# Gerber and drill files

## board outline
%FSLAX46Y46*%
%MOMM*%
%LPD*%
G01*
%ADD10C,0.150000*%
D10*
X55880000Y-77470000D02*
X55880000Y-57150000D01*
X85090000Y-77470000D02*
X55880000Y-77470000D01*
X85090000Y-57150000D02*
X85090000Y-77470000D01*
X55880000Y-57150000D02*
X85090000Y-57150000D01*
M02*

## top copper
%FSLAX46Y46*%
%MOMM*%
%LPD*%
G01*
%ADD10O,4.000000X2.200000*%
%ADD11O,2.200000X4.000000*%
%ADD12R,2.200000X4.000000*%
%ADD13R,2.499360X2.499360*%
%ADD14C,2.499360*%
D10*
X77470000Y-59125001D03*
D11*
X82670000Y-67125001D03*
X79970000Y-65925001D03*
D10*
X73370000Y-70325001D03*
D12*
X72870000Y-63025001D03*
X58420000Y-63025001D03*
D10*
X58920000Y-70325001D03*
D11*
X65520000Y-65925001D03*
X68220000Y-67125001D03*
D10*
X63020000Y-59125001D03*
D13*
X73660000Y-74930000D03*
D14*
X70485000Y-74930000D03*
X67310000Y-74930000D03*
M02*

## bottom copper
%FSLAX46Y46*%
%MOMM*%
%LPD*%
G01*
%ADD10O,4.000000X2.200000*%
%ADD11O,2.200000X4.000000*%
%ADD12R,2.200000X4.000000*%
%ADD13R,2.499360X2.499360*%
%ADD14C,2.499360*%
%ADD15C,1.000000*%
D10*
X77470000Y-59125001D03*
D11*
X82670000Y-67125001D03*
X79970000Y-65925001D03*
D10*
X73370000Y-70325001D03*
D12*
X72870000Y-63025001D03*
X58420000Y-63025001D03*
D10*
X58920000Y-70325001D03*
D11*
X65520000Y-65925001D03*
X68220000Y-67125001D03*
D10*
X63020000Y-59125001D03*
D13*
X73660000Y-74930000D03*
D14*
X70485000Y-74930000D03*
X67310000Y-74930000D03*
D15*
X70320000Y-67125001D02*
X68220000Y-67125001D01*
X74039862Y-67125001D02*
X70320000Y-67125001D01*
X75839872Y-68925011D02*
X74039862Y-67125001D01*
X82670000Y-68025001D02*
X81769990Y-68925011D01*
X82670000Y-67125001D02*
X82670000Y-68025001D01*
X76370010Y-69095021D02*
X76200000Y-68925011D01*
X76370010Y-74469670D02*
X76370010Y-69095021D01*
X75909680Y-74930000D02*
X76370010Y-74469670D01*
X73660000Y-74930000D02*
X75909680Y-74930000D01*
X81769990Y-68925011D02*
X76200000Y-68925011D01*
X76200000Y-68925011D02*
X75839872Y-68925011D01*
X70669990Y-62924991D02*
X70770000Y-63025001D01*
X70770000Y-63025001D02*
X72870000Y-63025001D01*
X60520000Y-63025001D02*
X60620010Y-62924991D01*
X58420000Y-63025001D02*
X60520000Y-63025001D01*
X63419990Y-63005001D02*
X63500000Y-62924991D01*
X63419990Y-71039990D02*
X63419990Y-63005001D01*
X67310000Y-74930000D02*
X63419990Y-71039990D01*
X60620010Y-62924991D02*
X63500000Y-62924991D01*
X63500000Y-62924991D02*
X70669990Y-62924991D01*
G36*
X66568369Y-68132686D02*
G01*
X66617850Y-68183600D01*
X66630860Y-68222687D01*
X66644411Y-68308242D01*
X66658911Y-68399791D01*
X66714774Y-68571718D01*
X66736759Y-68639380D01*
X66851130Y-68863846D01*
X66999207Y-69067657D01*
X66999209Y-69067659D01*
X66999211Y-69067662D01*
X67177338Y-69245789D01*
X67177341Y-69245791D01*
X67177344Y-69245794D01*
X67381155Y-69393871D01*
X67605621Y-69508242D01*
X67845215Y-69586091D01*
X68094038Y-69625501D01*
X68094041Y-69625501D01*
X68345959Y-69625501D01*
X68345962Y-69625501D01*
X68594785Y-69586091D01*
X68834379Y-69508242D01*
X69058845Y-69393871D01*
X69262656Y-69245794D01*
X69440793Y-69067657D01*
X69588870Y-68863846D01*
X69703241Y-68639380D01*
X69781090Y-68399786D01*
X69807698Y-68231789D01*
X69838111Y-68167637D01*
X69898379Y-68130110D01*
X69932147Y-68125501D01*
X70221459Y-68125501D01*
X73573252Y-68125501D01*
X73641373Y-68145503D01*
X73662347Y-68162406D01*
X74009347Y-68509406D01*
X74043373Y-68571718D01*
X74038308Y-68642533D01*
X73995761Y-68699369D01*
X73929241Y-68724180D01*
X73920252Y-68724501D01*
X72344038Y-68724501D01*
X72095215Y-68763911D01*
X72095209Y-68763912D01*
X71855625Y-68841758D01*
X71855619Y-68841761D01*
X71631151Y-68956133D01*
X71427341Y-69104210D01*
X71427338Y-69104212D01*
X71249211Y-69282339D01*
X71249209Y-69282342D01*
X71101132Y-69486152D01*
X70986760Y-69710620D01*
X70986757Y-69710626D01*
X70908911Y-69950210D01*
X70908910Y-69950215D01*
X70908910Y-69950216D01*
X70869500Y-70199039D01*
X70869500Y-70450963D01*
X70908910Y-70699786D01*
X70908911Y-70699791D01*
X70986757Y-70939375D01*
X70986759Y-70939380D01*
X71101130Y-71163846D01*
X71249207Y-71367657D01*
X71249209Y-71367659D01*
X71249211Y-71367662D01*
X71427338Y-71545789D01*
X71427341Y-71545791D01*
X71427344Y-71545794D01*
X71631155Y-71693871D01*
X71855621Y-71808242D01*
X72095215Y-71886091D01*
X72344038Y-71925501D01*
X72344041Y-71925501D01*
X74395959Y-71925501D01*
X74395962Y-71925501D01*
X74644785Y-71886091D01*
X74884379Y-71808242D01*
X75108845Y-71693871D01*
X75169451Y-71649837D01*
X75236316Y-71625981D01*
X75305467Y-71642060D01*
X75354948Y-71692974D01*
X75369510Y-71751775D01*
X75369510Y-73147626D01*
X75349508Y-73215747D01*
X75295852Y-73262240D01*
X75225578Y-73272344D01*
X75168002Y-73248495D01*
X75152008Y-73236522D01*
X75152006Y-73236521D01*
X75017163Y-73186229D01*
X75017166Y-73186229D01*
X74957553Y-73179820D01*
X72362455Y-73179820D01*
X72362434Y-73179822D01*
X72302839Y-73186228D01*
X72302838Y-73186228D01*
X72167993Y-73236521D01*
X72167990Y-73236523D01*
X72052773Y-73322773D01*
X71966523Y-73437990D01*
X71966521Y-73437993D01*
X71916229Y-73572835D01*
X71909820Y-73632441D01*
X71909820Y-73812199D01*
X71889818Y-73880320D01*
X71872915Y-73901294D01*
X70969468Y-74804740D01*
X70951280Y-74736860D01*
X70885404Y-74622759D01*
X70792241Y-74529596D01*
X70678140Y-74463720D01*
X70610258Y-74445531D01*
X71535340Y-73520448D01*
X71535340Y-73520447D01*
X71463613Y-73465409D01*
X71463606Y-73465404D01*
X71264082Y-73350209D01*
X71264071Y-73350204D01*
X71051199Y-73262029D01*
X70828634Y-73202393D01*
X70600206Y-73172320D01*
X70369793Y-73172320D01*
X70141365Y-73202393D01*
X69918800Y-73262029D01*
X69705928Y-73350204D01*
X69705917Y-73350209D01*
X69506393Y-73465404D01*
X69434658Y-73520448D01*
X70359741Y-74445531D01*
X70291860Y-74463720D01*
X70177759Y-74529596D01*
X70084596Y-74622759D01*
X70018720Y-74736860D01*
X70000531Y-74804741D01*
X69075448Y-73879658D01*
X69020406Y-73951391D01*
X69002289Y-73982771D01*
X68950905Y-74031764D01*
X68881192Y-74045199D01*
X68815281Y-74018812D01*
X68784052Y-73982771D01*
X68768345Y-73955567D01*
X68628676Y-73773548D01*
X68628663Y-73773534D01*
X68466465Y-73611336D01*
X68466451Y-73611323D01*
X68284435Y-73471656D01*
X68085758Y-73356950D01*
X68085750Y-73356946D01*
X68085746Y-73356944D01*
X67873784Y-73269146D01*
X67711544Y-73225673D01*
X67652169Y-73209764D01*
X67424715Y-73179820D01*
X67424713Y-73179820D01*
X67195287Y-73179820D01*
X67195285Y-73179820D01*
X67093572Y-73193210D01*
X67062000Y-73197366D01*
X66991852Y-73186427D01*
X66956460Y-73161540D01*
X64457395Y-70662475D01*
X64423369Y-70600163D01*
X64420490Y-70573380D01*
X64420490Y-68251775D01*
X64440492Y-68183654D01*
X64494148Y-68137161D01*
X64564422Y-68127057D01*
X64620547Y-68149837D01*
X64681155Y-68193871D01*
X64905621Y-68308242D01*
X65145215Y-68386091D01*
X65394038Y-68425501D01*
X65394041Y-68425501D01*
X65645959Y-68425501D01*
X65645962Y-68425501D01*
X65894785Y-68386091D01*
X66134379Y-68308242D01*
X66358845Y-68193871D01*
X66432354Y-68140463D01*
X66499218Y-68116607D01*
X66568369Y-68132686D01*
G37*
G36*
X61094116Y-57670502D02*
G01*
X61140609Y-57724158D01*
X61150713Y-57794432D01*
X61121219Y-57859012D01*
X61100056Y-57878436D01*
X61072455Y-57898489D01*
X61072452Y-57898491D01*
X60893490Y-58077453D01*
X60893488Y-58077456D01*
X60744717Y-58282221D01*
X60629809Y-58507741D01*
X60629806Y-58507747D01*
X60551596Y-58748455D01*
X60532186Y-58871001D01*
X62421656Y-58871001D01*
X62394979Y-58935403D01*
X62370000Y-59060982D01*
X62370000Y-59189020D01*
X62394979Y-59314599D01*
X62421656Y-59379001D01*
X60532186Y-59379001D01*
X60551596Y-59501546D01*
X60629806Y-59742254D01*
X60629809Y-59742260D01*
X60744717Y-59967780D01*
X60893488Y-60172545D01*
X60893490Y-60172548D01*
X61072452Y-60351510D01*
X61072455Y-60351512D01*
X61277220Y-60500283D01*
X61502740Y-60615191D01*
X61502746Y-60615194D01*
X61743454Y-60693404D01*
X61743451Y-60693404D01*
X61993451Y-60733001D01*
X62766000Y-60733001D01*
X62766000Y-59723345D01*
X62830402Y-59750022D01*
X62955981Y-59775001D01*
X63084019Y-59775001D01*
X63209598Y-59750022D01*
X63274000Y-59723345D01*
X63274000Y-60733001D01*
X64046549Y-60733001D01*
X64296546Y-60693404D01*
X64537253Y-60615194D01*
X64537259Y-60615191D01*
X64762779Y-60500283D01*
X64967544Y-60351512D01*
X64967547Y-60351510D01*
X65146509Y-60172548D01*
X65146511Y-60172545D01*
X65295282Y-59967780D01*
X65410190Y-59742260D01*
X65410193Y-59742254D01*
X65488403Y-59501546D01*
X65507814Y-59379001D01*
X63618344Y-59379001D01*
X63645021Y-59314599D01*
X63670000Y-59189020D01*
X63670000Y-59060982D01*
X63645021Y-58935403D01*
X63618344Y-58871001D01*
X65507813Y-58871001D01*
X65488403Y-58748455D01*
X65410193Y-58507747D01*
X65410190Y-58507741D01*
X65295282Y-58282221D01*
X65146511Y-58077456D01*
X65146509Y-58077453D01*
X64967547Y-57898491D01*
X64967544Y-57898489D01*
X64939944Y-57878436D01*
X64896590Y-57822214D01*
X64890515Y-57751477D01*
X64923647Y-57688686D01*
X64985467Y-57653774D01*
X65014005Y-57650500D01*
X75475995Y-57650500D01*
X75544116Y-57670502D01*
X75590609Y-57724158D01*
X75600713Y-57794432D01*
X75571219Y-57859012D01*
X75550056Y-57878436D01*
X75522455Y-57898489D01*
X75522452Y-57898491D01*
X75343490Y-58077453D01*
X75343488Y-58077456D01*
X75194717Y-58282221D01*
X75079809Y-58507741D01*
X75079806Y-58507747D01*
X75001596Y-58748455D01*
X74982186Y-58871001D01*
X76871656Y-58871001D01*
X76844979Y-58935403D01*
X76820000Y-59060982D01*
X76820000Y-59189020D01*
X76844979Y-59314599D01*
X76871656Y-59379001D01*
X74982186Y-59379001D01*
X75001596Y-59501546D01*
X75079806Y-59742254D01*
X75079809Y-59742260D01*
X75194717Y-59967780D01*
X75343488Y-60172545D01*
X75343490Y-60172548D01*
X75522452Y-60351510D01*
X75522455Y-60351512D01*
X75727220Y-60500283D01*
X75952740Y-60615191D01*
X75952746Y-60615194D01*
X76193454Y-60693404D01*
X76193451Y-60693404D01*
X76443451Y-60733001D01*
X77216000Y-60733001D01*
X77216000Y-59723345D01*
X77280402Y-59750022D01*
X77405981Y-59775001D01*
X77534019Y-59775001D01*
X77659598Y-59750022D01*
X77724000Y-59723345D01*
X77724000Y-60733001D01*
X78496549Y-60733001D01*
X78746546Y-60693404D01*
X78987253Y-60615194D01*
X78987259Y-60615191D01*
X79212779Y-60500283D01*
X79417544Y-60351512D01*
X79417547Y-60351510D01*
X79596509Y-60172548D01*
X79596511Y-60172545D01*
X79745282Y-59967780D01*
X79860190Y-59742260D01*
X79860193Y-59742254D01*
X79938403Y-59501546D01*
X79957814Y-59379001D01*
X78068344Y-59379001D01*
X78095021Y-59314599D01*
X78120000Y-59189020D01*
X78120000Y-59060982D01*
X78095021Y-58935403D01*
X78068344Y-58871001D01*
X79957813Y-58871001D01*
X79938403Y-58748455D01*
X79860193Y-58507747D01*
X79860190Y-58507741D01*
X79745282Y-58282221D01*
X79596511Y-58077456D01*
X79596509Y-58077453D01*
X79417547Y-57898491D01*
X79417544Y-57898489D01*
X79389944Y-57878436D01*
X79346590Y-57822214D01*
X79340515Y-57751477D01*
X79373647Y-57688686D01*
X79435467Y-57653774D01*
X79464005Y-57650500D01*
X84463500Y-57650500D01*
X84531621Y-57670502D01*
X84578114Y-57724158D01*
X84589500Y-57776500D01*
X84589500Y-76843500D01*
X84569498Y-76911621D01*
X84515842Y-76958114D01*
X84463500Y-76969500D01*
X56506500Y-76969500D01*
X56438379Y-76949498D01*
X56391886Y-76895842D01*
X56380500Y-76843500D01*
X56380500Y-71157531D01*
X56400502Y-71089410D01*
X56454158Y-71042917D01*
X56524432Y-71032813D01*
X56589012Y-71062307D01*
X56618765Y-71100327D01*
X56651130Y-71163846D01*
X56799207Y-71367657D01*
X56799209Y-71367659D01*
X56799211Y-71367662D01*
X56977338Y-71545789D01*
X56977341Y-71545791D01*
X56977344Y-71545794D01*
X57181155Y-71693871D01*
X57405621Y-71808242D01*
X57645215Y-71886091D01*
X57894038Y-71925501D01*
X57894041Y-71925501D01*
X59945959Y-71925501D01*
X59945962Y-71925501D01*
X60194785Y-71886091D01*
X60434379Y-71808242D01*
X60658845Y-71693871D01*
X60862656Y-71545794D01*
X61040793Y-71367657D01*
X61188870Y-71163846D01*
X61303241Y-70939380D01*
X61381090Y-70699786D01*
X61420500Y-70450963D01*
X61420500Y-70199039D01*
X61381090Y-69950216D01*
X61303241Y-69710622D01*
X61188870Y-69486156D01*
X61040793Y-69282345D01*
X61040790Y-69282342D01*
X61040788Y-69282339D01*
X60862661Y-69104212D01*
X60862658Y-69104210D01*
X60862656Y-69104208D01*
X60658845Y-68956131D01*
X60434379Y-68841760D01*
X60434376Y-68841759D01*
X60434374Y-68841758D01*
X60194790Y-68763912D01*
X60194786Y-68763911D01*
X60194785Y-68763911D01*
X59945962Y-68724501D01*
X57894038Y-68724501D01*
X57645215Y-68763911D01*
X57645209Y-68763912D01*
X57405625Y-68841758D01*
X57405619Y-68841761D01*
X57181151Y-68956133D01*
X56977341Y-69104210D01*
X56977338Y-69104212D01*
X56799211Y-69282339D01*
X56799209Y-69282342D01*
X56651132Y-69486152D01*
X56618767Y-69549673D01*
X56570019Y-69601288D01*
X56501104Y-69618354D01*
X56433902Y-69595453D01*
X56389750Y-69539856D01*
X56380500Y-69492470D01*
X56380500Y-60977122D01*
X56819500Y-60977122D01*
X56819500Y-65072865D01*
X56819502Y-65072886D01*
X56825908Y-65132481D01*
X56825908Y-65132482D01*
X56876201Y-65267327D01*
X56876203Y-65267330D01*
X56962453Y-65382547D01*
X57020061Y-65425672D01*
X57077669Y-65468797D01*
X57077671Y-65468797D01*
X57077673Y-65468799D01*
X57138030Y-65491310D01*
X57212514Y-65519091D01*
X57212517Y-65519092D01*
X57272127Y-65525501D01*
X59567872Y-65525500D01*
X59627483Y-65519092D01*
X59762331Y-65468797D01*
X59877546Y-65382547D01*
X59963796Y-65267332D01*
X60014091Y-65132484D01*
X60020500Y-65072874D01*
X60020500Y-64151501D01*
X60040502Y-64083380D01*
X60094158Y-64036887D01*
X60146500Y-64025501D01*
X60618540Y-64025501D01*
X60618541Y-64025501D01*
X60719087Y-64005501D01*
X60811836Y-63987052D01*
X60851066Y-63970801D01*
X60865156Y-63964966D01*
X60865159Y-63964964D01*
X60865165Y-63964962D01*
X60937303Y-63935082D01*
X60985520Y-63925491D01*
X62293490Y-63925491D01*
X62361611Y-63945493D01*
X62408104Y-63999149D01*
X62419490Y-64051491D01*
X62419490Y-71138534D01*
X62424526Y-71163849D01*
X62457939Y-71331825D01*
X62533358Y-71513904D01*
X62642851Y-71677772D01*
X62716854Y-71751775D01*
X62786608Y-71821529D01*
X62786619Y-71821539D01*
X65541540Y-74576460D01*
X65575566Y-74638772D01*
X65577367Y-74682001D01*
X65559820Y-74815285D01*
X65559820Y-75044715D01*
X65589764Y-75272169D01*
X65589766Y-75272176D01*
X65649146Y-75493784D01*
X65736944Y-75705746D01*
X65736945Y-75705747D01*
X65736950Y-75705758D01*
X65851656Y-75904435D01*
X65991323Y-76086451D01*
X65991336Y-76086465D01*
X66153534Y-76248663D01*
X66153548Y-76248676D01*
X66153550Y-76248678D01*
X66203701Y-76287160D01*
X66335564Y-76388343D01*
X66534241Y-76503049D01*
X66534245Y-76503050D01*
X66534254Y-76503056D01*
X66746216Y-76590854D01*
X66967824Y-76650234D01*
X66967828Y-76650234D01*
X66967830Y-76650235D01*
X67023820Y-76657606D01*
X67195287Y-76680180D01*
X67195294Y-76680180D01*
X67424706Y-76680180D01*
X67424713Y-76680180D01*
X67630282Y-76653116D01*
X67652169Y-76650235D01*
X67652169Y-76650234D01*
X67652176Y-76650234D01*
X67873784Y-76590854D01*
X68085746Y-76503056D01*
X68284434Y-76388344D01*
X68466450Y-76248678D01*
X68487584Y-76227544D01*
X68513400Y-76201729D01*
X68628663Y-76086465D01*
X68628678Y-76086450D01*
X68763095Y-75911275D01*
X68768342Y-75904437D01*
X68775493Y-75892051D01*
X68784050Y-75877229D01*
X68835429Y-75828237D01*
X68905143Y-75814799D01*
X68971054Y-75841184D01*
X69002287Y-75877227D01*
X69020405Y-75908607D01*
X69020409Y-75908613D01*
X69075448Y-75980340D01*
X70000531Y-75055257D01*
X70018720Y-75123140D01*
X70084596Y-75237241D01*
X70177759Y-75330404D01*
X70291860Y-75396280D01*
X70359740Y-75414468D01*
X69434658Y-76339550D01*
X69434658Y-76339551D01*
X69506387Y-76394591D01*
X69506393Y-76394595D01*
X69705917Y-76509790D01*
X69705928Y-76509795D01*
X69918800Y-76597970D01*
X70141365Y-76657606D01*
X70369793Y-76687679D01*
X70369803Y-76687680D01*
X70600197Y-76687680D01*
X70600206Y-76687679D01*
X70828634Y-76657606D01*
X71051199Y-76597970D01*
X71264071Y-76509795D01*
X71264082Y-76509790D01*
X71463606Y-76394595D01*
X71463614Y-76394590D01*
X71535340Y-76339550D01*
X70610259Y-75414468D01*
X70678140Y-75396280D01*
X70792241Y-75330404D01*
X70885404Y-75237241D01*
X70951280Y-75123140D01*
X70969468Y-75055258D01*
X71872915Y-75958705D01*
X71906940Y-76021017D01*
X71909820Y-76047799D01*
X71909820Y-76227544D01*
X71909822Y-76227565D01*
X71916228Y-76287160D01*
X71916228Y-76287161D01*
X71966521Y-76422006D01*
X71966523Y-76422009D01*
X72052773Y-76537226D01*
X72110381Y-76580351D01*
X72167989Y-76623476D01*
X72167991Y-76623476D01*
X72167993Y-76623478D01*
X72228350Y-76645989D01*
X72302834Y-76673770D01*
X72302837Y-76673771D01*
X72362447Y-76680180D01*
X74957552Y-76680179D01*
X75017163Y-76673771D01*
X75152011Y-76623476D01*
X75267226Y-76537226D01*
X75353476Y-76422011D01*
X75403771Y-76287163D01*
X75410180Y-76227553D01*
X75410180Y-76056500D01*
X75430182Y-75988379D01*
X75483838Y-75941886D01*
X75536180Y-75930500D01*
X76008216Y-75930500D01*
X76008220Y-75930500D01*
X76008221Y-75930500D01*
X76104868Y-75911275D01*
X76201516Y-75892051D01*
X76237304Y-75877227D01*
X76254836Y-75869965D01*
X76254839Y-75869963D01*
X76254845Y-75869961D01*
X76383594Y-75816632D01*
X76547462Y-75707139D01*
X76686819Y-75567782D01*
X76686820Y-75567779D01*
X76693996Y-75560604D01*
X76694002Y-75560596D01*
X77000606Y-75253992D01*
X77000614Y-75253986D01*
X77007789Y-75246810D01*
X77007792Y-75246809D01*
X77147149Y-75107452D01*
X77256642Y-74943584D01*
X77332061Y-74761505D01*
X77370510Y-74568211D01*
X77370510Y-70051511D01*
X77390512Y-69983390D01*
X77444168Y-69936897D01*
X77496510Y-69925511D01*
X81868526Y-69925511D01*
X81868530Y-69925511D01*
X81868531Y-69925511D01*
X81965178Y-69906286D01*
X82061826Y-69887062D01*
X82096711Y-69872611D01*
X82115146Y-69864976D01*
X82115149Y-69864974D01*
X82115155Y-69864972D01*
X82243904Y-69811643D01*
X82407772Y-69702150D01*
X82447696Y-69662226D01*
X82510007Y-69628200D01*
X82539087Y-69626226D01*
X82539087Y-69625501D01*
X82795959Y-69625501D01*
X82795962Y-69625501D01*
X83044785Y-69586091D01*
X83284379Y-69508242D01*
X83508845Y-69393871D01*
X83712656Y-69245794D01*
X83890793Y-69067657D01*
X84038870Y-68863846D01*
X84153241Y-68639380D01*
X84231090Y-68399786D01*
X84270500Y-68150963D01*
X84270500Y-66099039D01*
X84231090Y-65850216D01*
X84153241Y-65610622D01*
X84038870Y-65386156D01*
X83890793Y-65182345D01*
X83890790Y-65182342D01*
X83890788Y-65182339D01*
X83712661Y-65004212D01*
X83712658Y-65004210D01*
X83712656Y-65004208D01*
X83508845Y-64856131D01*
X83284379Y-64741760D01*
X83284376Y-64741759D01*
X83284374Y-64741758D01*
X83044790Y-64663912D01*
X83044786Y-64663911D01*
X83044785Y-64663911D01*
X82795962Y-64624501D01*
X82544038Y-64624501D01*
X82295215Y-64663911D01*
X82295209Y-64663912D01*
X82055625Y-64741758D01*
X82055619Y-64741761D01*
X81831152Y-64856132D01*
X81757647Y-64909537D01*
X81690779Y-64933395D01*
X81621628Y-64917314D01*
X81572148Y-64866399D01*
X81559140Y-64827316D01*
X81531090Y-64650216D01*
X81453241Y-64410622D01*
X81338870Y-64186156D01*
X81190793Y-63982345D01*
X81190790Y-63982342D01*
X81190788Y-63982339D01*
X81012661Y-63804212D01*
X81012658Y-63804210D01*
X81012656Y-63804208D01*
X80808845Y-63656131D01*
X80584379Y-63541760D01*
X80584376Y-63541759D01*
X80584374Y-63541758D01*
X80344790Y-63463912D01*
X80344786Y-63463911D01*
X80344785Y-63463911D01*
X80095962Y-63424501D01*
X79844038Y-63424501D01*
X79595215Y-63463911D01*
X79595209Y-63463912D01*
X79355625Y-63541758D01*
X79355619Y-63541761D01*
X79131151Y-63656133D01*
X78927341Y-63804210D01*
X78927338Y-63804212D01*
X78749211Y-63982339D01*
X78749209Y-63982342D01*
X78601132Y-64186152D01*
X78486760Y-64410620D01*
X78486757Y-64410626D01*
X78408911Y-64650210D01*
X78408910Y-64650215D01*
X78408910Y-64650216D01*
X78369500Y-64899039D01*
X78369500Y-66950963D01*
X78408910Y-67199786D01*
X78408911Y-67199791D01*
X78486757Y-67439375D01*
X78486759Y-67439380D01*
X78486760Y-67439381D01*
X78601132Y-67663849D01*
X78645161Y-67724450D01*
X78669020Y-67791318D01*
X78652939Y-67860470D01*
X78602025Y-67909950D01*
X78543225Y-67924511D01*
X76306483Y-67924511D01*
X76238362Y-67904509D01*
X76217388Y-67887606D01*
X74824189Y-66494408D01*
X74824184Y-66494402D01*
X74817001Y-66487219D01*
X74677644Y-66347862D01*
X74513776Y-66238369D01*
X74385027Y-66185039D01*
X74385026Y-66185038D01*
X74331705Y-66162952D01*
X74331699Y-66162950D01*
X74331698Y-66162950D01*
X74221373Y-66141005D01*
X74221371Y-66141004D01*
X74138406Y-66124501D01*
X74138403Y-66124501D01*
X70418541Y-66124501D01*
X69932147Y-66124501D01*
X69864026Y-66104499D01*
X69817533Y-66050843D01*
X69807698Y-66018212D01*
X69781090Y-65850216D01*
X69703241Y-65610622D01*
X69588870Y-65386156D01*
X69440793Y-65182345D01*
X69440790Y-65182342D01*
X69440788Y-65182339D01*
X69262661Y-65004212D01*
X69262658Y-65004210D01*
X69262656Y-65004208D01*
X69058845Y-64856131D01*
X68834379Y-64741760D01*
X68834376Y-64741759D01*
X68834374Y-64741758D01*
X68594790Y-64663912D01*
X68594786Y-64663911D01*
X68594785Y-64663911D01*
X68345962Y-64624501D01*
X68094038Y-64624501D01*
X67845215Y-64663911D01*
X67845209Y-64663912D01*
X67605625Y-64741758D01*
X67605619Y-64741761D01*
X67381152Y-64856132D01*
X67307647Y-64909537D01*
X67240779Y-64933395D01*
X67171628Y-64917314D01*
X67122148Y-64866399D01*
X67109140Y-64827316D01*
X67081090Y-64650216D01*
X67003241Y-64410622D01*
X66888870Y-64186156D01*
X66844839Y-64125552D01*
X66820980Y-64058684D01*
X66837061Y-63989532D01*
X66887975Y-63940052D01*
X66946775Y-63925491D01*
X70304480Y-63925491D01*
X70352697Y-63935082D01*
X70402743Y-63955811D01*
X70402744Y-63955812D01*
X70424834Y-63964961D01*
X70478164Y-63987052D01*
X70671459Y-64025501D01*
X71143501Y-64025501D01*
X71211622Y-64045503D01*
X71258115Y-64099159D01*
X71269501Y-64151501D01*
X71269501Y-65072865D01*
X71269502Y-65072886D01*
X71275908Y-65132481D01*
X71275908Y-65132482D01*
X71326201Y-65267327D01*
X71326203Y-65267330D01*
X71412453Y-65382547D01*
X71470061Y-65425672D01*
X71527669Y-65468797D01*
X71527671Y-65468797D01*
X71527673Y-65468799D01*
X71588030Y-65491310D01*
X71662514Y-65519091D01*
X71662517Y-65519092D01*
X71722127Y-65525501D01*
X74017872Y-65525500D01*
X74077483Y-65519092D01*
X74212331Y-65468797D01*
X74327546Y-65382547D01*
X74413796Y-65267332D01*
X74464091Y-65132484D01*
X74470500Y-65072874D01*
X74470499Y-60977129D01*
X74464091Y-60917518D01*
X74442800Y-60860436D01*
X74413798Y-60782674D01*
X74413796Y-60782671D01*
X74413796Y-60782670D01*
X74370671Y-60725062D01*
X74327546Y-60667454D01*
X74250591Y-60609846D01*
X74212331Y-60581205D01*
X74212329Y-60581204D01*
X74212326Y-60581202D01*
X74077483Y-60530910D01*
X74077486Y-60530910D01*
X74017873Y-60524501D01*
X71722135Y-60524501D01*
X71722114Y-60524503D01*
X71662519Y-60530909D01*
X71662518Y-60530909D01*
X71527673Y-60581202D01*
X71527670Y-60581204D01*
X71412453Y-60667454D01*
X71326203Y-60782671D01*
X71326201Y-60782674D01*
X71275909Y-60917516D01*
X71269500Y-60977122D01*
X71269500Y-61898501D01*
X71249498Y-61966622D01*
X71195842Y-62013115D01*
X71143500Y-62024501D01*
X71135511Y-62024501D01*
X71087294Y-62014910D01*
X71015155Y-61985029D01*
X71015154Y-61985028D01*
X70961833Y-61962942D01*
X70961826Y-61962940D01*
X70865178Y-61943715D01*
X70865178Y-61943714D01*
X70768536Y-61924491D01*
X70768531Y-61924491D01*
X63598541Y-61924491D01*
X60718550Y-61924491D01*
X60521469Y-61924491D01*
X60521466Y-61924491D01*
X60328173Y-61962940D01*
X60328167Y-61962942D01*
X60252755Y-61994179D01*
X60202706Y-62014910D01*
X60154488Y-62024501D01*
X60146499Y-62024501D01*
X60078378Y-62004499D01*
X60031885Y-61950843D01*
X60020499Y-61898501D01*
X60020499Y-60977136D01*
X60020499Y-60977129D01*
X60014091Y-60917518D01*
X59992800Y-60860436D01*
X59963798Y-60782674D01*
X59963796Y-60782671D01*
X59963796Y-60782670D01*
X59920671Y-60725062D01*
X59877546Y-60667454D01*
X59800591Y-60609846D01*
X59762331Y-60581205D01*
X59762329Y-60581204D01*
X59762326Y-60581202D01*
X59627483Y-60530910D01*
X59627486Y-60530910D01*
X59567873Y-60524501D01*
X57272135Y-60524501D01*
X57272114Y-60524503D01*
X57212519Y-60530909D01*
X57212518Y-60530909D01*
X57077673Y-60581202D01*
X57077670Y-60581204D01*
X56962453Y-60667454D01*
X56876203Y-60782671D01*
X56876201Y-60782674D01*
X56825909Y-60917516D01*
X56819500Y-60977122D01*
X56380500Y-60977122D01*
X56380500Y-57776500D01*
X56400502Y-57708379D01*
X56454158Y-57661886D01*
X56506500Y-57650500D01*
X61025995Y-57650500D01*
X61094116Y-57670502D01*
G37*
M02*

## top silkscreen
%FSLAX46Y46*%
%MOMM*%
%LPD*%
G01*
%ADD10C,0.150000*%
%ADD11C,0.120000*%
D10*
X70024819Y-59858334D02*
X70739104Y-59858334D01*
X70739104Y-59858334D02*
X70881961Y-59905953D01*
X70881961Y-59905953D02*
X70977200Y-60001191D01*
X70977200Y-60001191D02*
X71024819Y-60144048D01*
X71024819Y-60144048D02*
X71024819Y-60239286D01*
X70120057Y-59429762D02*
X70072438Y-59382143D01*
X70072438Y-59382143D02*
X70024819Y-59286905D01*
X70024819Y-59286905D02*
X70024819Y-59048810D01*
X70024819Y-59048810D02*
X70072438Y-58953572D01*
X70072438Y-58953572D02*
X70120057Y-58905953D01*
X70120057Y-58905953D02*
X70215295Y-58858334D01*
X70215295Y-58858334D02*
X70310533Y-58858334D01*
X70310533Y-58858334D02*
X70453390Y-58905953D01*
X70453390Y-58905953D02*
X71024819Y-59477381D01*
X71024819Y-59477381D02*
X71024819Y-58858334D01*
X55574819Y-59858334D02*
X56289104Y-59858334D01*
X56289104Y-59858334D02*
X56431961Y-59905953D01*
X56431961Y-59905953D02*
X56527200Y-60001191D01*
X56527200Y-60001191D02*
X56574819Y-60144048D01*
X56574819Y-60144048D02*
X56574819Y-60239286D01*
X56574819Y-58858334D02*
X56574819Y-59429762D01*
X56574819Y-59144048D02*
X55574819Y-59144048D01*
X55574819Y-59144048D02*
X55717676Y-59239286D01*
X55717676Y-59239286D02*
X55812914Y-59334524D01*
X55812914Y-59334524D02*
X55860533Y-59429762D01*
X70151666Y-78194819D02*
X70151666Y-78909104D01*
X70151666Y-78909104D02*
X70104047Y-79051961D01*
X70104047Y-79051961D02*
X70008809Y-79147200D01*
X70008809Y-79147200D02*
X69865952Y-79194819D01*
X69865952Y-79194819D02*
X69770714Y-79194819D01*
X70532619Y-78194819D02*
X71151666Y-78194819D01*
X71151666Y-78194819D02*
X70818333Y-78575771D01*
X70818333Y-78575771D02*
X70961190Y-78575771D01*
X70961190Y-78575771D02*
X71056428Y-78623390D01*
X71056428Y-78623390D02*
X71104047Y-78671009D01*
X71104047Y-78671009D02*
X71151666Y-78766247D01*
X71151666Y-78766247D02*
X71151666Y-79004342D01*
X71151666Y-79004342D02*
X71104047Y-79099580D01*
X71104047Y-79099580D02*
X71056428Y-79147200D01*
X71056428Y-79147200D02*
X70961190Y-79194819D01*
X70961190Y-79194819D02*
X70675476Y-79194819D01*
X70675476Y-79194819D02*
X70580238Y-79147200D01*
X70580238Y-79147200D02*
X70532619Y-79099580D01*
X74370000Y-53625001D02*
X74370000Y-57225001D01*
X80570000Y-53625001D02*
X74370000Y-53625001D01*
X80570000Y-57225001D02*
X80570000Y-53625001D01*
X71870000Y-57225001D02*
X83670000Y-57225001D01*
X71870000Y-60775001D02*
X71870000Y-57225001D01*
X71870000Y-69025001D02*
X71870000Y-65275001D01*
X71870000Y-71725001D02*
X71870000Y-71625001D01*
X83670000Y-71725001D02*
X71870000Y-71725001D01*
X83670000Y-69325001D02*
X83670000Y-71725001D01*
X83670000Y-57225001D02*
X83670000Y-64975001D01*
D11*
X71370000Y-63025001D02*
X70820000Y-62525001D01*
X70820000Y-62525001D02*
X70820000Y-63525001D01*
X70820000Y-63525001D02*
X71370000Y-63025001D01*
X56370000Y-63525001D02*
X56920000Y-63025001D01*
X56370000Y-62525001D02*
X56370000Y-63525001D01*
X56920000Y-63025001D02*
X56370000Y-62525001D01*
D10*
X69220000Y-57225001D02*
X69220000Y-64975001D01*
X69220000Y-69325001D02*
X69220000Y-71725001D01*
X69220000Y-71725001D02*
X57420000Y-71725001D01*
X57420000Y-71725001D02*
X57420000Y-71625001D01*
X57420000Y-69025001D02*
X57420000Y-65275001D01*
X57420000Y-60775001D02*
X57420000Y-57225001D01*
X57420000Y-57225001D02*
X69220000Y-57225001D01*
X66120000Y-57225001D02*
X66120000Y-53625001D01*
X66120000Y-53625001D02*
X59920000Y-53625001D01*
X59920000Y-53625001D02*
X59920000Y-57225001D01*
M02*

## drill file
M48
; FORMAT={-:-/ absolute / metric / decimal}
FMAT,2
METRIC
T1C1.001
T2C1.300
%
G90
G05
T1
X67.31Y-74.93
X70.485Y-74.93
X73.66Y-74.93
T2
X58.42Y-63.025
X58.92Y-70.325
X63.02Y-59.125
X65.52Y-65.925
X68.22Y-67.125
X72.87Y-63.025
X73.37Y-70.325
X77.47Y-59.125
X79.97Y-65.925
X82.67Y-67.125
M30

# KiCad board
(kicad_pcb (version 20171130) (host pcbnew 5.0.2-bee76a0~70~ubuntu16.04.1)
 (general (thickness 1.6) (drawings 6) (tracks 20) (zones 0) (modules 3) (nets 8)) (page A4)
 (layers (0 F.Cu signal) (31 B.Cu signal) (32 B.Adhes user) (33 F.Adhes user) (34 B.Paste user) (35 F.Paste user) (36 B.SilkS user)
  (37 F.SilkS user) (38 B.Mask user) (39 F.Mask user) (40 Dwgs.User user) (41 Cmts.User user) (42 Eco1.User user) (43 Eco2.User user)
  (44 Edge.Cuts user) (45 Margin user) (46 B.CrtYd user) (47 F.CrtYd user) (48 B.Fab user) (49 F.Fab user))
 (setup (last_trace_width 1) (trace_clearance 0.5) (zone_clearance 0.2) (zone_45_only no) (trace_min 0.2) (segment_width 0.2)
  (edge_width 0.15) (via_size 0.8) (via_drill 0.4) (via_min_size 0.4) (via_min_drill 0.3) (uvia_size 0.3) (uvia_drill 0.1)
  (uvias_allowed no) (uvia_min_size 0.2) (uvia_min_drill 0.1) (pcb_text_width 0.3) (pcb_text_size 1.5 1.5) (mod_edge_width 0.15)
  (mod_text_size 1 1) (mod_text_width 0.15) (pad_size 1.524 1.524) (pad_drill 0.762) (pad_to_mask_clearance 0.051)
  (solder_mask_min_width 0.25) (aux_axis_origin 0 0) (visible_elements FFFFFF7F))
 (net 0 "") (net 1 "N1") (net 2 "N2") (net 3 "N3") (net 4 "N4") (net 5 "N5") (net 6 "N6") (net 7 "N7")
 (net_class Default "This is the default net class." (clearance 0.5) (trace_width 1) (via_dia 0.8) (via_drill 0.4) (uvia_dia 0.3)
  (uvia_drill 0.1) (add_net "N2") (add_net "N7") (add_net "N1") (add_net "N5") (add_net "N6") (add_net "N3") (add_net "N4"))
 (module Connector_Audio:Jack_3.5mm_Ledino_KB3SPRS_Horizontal (layer F.Cu) (at 72.87 63.025001 270)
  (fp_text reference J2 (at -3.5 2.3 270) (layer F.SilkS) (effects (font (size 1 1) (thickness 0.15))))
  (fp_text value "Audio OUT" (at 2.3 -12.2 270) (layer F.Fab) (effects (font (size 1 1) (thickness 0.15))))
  (fp_line (start -9.4 -1.5) (end -5.8 -1.5) (layer F.SilkS) (width 0.15))
  (fp_line (start -9.4 -7.7) (end -9.4 -1.5) (layer F.SilkS) (width 0.15))
  (fp_line (start -5.8 -7.7) (end -9.4 -7.7) (layer F.SilkS) (width 0.15))
  (fp_line (start -5.8 1) (end -5.8 -10.8) (layer F.SilkS) (width 0.15))
  (fp_line (start -2.25 1) (end -5.8 1) (layer F.SilkS) (width 0.15))
  (fp_line (start 6 1) (end 2.25 1) (layer F.SilkS) (width 0.15))
  (fp_line (start 8.7 1) (end 8.6 1) (layer F.SilkS) (width 0.15))
  (fp_line (start 8.7 -10.8) (end 8.7 1) (layer F.SilkS) (width 0.15))
  (fp_line (start 6.3 -10.8) (end 8.7 -10.8) (layer F.SilkS) (width 0.15))
  (fp_line (start -5.8 -10.8) (end 1.95 -10.8) (layer F.SilkS) (width 0.15))
  (fp_line (start 0 1.5) (end -0.5 2.05) (layer F.SilkS) (width 0.12))
  (fp_line (start -0.5 2.05) (end 0.5 2.05) (layer F.SilkS) (width 0.12))
  (fp_line (start 0.5 2.05) (end 0 1.5) (layer F.SilkS) (width 0.12))
  (pad S thru_hole oval (at -3.9 -4.6 270) (size 2.2 4) (drill 1.3) (layers *.Cu *.Mask) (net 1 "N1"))
  (pad R thru_hole oval (at 4.1 -9.8 270) (size 4 2.2) (drill 1.3) (layers *.Cu *.Mask) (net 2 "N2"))
  (pad RN thru_hole oval (at 2.9 -7.1 270) (size 4 2.2) (drill 1.3) (layers *.Cu *.Mask) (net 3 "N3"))
  (pad TN thru_hole oval (at 7.3 -0.5) (size 4 2.2) (drill 1.3) (layers *.Cu *.Mask) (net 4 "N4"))
  (pad T thru_hole rect (at 0 0 270) (size 4 2.2) (drill 1.3) (layers *.Cu *.Mask) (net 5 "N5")))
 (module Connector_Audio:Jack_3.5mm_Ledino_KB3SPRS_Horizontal (layer F.Cu) (at 58.42 63.025001 270)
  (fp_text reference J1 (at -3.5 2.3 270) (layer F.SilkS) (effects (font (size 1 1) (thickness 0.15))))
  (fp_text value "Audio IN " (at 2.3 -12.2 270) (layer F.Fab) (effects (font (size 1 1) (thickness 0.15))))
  (fp_line (start 0.5 2.05) (end 0 1.5) (layer F.SilkS) (width 0.12))
  (fp_line (start -0.5 2.05) (end 0.5 2.05) (layer F.SilkS) (width 0.12))
  (fp_line (start 0 1.5) (end -0.5 2.05) (layer F.SilkS) (width 0.12))
  (fp_line (start -5.8 -10.8) (end 1.95 -10.8) (layer F.SilkS) (width 0.15))
  (fp_line (start 6.3 -10.8) (end 8.7 -10.8) (layer F.SilkS) (width 0.15))
  (fp_line (start 8.7 -10.8) (end 8.7 1) (layer F.SilkS) (width 0.15))
  (fp_line (start 8.7 1) (end 8.6 1) (layer F.SilkS) (width 0.15))
  (fp_line (start 6 1) (end 2.25 1) (layer F.SilkS) (width 0.15))
  (fp_line (start -2.25 1) (end -5.8 1) (layer F.SilkS) (width 0.15))
  (fp_line (start -5.8 1) (end -5.8 -10.8) (layer F.SilkS) (width 0.15))
  (fp_line (start -5.8 -7.7) (end -9.4 -7.7) (layer F.SilkS) (width 0.15))
  (fp_line (start -9.4 -7.7) (end -9.4 -1.5) (layer F.SilkS) (width 0.15))
  (fp_line (start -9.4 -1.5) (end -5.8 -1.5) (layer F.SilkS) (width 0.15))
  (pad T thru_hole rect (at 0 0 270) (size 4 2.2) (drill 1.3) (layers *.Cu *.Mask) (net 5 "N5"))
  (pad TN thru_hole oval (at 7.3 -0.5) (size 4 2.2) (drill 1.3) (layers *.Cu *.Mask) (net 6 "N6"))
  (pad RN thru_hole oval (at 2.9 -7.1 270) (size 4 2.2) (drill 1.3) (layers *.Cu *.Mask) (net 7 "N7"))
  (pad R thru_hole oval (at 4.1 -9.8 270) (size 4 2.2) (drill 1.3) (layers *.Cu *.Mask) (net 2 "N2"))
  (pad S thru_hole oval (at -3.9 -4.6 270) (size 2.2 4) (drill 1.3) (layers *.Cu *.Mask) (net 1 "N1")))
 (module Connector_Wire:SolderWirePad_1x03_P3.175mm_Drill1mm (layer F.Cu) (at 73.66 74.93 180)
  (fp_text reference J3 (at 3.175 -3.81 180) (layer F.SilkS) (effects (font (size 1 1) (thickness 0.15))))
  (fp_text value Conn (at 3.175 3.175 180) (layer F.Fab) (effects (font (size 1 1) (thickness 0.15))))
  (pad 1 thru_hole rect (at 0 0 180) (size 2.49936 2.49936) (drill 1.00076) (layers *.Cu *.Mask) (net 2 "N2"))
  (pad 2 thru_hole circle (at 3.175 0 180) (size 2.49936 2.49936) (drill 1.00076) (layers *.Cu *.Mask) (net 1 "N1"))
  (pad 3 thru_hole circle (at 6.35 0 180) (size 2.49936 2.49936) (drill 1.00076) (layers *.Cu *.Mask) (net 5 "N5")))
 (gr_line (start 55.88 77.47) (end 55.88 57.15) (layer Edge.Cuts) (width 0.15))
 (gr_line (start 85.09 77.47) (end 55.88 77.47) (layer Edge.Cuts) (width 0.15))
 (gr_line (start 85.09 57.15) (end 85.09 77.47) (layer Edge.Cuts) (width 0.15))
 (gr_line (start 55.88 57.15) (end 85.09 57.15) (layer Edge.Cuts) (width 0.15))
 (segment (start 70.32 67.125001) (end 68.22 67.125001) (width 1) (layer B.Cu) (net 2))
 (segment (start 74.039862 67.125001) (end 70.32 67.125001) (width 1) (layer B.Cu) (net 2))
 (segment (start 75.839872 68.925011) (end 74.039862 67.125001) (width 1) (layer B.Cu) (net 2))
 (segment (start 82.67 68.025001) (end 81.76999 68.925011) (width 1) (layer B.Cu) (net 2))
 (segment (start 82.67 67.125001) (end 82.67 68.025001) (width 1) (layer B.Cu) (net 2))
 (segment (start 76.37001 69.095021) (end 76.2 68.925011) (width 1) (layer B.Cu) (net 2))
 (segment (start 76.37001 74.46967) (end 76.37001 69.095021) (width 1) (layer B.Cu) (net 2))
 (segment (start 75.90968 74.93) (end 76.37001 74.46967) (width 1) (layer B.Cu) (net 2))
 (segment (start 73.66 74.93) (end 75.90968 74.93) (width 1) (layer B.Cu) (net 2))
 (segment (start 81.76999 68.925011) (end 76.2 68.925011) (width 1) (layer B.Cu) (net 2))
 (segment (start 76.2 68.925011) (end 75.839872 68.925011) (width 1) (layer B.Cu) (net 2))
 (segment (start 70.66999 62.924991) (end 70.77 63.025001) (width 1) (layer B.Cu) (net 5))
 (segment (start 70.77 63.025001) (end 72.87 63.025001) (width 1) (layer B.Cu) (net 5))
 (segment (start 60.52 63.025001) (end 60.62001 62.924991) (width 1) (layer B.Cu) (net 5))
 (segment (start 58.42 63.025001) (end 60.52 63.025001) (width 1) (layer B.Cu) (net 5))
 (segment (start 63.41999 63.005001) (end 63.5 62.924991) (width 1) (layer B.Cu) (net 5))
 (segment (start 63.41999 71.03999) (end 63.41999 63.005001) (width 1) (layer B.Cu) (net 5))
 (segment (start 67.31 74.93) (end 63.41999 71.03999) (width 1) (layer B.Cu) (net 5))
 (segment (start 60.62001 62.924991) (end 63.5 62.924991) (width 1) (layer B.Cu) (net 5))
 (segment (start 63.5 62.924991) (end 70.66999 62.924991) (width 1) (layer B.Cu) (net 5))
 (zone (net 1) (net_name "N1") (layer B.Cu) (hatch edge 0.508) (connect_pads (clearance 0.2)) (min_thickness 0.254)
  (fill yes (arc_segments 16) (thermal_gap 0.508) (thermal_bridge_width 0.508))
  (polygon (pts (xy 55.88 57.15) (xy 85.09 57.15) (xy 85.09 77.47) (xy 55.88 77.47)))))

